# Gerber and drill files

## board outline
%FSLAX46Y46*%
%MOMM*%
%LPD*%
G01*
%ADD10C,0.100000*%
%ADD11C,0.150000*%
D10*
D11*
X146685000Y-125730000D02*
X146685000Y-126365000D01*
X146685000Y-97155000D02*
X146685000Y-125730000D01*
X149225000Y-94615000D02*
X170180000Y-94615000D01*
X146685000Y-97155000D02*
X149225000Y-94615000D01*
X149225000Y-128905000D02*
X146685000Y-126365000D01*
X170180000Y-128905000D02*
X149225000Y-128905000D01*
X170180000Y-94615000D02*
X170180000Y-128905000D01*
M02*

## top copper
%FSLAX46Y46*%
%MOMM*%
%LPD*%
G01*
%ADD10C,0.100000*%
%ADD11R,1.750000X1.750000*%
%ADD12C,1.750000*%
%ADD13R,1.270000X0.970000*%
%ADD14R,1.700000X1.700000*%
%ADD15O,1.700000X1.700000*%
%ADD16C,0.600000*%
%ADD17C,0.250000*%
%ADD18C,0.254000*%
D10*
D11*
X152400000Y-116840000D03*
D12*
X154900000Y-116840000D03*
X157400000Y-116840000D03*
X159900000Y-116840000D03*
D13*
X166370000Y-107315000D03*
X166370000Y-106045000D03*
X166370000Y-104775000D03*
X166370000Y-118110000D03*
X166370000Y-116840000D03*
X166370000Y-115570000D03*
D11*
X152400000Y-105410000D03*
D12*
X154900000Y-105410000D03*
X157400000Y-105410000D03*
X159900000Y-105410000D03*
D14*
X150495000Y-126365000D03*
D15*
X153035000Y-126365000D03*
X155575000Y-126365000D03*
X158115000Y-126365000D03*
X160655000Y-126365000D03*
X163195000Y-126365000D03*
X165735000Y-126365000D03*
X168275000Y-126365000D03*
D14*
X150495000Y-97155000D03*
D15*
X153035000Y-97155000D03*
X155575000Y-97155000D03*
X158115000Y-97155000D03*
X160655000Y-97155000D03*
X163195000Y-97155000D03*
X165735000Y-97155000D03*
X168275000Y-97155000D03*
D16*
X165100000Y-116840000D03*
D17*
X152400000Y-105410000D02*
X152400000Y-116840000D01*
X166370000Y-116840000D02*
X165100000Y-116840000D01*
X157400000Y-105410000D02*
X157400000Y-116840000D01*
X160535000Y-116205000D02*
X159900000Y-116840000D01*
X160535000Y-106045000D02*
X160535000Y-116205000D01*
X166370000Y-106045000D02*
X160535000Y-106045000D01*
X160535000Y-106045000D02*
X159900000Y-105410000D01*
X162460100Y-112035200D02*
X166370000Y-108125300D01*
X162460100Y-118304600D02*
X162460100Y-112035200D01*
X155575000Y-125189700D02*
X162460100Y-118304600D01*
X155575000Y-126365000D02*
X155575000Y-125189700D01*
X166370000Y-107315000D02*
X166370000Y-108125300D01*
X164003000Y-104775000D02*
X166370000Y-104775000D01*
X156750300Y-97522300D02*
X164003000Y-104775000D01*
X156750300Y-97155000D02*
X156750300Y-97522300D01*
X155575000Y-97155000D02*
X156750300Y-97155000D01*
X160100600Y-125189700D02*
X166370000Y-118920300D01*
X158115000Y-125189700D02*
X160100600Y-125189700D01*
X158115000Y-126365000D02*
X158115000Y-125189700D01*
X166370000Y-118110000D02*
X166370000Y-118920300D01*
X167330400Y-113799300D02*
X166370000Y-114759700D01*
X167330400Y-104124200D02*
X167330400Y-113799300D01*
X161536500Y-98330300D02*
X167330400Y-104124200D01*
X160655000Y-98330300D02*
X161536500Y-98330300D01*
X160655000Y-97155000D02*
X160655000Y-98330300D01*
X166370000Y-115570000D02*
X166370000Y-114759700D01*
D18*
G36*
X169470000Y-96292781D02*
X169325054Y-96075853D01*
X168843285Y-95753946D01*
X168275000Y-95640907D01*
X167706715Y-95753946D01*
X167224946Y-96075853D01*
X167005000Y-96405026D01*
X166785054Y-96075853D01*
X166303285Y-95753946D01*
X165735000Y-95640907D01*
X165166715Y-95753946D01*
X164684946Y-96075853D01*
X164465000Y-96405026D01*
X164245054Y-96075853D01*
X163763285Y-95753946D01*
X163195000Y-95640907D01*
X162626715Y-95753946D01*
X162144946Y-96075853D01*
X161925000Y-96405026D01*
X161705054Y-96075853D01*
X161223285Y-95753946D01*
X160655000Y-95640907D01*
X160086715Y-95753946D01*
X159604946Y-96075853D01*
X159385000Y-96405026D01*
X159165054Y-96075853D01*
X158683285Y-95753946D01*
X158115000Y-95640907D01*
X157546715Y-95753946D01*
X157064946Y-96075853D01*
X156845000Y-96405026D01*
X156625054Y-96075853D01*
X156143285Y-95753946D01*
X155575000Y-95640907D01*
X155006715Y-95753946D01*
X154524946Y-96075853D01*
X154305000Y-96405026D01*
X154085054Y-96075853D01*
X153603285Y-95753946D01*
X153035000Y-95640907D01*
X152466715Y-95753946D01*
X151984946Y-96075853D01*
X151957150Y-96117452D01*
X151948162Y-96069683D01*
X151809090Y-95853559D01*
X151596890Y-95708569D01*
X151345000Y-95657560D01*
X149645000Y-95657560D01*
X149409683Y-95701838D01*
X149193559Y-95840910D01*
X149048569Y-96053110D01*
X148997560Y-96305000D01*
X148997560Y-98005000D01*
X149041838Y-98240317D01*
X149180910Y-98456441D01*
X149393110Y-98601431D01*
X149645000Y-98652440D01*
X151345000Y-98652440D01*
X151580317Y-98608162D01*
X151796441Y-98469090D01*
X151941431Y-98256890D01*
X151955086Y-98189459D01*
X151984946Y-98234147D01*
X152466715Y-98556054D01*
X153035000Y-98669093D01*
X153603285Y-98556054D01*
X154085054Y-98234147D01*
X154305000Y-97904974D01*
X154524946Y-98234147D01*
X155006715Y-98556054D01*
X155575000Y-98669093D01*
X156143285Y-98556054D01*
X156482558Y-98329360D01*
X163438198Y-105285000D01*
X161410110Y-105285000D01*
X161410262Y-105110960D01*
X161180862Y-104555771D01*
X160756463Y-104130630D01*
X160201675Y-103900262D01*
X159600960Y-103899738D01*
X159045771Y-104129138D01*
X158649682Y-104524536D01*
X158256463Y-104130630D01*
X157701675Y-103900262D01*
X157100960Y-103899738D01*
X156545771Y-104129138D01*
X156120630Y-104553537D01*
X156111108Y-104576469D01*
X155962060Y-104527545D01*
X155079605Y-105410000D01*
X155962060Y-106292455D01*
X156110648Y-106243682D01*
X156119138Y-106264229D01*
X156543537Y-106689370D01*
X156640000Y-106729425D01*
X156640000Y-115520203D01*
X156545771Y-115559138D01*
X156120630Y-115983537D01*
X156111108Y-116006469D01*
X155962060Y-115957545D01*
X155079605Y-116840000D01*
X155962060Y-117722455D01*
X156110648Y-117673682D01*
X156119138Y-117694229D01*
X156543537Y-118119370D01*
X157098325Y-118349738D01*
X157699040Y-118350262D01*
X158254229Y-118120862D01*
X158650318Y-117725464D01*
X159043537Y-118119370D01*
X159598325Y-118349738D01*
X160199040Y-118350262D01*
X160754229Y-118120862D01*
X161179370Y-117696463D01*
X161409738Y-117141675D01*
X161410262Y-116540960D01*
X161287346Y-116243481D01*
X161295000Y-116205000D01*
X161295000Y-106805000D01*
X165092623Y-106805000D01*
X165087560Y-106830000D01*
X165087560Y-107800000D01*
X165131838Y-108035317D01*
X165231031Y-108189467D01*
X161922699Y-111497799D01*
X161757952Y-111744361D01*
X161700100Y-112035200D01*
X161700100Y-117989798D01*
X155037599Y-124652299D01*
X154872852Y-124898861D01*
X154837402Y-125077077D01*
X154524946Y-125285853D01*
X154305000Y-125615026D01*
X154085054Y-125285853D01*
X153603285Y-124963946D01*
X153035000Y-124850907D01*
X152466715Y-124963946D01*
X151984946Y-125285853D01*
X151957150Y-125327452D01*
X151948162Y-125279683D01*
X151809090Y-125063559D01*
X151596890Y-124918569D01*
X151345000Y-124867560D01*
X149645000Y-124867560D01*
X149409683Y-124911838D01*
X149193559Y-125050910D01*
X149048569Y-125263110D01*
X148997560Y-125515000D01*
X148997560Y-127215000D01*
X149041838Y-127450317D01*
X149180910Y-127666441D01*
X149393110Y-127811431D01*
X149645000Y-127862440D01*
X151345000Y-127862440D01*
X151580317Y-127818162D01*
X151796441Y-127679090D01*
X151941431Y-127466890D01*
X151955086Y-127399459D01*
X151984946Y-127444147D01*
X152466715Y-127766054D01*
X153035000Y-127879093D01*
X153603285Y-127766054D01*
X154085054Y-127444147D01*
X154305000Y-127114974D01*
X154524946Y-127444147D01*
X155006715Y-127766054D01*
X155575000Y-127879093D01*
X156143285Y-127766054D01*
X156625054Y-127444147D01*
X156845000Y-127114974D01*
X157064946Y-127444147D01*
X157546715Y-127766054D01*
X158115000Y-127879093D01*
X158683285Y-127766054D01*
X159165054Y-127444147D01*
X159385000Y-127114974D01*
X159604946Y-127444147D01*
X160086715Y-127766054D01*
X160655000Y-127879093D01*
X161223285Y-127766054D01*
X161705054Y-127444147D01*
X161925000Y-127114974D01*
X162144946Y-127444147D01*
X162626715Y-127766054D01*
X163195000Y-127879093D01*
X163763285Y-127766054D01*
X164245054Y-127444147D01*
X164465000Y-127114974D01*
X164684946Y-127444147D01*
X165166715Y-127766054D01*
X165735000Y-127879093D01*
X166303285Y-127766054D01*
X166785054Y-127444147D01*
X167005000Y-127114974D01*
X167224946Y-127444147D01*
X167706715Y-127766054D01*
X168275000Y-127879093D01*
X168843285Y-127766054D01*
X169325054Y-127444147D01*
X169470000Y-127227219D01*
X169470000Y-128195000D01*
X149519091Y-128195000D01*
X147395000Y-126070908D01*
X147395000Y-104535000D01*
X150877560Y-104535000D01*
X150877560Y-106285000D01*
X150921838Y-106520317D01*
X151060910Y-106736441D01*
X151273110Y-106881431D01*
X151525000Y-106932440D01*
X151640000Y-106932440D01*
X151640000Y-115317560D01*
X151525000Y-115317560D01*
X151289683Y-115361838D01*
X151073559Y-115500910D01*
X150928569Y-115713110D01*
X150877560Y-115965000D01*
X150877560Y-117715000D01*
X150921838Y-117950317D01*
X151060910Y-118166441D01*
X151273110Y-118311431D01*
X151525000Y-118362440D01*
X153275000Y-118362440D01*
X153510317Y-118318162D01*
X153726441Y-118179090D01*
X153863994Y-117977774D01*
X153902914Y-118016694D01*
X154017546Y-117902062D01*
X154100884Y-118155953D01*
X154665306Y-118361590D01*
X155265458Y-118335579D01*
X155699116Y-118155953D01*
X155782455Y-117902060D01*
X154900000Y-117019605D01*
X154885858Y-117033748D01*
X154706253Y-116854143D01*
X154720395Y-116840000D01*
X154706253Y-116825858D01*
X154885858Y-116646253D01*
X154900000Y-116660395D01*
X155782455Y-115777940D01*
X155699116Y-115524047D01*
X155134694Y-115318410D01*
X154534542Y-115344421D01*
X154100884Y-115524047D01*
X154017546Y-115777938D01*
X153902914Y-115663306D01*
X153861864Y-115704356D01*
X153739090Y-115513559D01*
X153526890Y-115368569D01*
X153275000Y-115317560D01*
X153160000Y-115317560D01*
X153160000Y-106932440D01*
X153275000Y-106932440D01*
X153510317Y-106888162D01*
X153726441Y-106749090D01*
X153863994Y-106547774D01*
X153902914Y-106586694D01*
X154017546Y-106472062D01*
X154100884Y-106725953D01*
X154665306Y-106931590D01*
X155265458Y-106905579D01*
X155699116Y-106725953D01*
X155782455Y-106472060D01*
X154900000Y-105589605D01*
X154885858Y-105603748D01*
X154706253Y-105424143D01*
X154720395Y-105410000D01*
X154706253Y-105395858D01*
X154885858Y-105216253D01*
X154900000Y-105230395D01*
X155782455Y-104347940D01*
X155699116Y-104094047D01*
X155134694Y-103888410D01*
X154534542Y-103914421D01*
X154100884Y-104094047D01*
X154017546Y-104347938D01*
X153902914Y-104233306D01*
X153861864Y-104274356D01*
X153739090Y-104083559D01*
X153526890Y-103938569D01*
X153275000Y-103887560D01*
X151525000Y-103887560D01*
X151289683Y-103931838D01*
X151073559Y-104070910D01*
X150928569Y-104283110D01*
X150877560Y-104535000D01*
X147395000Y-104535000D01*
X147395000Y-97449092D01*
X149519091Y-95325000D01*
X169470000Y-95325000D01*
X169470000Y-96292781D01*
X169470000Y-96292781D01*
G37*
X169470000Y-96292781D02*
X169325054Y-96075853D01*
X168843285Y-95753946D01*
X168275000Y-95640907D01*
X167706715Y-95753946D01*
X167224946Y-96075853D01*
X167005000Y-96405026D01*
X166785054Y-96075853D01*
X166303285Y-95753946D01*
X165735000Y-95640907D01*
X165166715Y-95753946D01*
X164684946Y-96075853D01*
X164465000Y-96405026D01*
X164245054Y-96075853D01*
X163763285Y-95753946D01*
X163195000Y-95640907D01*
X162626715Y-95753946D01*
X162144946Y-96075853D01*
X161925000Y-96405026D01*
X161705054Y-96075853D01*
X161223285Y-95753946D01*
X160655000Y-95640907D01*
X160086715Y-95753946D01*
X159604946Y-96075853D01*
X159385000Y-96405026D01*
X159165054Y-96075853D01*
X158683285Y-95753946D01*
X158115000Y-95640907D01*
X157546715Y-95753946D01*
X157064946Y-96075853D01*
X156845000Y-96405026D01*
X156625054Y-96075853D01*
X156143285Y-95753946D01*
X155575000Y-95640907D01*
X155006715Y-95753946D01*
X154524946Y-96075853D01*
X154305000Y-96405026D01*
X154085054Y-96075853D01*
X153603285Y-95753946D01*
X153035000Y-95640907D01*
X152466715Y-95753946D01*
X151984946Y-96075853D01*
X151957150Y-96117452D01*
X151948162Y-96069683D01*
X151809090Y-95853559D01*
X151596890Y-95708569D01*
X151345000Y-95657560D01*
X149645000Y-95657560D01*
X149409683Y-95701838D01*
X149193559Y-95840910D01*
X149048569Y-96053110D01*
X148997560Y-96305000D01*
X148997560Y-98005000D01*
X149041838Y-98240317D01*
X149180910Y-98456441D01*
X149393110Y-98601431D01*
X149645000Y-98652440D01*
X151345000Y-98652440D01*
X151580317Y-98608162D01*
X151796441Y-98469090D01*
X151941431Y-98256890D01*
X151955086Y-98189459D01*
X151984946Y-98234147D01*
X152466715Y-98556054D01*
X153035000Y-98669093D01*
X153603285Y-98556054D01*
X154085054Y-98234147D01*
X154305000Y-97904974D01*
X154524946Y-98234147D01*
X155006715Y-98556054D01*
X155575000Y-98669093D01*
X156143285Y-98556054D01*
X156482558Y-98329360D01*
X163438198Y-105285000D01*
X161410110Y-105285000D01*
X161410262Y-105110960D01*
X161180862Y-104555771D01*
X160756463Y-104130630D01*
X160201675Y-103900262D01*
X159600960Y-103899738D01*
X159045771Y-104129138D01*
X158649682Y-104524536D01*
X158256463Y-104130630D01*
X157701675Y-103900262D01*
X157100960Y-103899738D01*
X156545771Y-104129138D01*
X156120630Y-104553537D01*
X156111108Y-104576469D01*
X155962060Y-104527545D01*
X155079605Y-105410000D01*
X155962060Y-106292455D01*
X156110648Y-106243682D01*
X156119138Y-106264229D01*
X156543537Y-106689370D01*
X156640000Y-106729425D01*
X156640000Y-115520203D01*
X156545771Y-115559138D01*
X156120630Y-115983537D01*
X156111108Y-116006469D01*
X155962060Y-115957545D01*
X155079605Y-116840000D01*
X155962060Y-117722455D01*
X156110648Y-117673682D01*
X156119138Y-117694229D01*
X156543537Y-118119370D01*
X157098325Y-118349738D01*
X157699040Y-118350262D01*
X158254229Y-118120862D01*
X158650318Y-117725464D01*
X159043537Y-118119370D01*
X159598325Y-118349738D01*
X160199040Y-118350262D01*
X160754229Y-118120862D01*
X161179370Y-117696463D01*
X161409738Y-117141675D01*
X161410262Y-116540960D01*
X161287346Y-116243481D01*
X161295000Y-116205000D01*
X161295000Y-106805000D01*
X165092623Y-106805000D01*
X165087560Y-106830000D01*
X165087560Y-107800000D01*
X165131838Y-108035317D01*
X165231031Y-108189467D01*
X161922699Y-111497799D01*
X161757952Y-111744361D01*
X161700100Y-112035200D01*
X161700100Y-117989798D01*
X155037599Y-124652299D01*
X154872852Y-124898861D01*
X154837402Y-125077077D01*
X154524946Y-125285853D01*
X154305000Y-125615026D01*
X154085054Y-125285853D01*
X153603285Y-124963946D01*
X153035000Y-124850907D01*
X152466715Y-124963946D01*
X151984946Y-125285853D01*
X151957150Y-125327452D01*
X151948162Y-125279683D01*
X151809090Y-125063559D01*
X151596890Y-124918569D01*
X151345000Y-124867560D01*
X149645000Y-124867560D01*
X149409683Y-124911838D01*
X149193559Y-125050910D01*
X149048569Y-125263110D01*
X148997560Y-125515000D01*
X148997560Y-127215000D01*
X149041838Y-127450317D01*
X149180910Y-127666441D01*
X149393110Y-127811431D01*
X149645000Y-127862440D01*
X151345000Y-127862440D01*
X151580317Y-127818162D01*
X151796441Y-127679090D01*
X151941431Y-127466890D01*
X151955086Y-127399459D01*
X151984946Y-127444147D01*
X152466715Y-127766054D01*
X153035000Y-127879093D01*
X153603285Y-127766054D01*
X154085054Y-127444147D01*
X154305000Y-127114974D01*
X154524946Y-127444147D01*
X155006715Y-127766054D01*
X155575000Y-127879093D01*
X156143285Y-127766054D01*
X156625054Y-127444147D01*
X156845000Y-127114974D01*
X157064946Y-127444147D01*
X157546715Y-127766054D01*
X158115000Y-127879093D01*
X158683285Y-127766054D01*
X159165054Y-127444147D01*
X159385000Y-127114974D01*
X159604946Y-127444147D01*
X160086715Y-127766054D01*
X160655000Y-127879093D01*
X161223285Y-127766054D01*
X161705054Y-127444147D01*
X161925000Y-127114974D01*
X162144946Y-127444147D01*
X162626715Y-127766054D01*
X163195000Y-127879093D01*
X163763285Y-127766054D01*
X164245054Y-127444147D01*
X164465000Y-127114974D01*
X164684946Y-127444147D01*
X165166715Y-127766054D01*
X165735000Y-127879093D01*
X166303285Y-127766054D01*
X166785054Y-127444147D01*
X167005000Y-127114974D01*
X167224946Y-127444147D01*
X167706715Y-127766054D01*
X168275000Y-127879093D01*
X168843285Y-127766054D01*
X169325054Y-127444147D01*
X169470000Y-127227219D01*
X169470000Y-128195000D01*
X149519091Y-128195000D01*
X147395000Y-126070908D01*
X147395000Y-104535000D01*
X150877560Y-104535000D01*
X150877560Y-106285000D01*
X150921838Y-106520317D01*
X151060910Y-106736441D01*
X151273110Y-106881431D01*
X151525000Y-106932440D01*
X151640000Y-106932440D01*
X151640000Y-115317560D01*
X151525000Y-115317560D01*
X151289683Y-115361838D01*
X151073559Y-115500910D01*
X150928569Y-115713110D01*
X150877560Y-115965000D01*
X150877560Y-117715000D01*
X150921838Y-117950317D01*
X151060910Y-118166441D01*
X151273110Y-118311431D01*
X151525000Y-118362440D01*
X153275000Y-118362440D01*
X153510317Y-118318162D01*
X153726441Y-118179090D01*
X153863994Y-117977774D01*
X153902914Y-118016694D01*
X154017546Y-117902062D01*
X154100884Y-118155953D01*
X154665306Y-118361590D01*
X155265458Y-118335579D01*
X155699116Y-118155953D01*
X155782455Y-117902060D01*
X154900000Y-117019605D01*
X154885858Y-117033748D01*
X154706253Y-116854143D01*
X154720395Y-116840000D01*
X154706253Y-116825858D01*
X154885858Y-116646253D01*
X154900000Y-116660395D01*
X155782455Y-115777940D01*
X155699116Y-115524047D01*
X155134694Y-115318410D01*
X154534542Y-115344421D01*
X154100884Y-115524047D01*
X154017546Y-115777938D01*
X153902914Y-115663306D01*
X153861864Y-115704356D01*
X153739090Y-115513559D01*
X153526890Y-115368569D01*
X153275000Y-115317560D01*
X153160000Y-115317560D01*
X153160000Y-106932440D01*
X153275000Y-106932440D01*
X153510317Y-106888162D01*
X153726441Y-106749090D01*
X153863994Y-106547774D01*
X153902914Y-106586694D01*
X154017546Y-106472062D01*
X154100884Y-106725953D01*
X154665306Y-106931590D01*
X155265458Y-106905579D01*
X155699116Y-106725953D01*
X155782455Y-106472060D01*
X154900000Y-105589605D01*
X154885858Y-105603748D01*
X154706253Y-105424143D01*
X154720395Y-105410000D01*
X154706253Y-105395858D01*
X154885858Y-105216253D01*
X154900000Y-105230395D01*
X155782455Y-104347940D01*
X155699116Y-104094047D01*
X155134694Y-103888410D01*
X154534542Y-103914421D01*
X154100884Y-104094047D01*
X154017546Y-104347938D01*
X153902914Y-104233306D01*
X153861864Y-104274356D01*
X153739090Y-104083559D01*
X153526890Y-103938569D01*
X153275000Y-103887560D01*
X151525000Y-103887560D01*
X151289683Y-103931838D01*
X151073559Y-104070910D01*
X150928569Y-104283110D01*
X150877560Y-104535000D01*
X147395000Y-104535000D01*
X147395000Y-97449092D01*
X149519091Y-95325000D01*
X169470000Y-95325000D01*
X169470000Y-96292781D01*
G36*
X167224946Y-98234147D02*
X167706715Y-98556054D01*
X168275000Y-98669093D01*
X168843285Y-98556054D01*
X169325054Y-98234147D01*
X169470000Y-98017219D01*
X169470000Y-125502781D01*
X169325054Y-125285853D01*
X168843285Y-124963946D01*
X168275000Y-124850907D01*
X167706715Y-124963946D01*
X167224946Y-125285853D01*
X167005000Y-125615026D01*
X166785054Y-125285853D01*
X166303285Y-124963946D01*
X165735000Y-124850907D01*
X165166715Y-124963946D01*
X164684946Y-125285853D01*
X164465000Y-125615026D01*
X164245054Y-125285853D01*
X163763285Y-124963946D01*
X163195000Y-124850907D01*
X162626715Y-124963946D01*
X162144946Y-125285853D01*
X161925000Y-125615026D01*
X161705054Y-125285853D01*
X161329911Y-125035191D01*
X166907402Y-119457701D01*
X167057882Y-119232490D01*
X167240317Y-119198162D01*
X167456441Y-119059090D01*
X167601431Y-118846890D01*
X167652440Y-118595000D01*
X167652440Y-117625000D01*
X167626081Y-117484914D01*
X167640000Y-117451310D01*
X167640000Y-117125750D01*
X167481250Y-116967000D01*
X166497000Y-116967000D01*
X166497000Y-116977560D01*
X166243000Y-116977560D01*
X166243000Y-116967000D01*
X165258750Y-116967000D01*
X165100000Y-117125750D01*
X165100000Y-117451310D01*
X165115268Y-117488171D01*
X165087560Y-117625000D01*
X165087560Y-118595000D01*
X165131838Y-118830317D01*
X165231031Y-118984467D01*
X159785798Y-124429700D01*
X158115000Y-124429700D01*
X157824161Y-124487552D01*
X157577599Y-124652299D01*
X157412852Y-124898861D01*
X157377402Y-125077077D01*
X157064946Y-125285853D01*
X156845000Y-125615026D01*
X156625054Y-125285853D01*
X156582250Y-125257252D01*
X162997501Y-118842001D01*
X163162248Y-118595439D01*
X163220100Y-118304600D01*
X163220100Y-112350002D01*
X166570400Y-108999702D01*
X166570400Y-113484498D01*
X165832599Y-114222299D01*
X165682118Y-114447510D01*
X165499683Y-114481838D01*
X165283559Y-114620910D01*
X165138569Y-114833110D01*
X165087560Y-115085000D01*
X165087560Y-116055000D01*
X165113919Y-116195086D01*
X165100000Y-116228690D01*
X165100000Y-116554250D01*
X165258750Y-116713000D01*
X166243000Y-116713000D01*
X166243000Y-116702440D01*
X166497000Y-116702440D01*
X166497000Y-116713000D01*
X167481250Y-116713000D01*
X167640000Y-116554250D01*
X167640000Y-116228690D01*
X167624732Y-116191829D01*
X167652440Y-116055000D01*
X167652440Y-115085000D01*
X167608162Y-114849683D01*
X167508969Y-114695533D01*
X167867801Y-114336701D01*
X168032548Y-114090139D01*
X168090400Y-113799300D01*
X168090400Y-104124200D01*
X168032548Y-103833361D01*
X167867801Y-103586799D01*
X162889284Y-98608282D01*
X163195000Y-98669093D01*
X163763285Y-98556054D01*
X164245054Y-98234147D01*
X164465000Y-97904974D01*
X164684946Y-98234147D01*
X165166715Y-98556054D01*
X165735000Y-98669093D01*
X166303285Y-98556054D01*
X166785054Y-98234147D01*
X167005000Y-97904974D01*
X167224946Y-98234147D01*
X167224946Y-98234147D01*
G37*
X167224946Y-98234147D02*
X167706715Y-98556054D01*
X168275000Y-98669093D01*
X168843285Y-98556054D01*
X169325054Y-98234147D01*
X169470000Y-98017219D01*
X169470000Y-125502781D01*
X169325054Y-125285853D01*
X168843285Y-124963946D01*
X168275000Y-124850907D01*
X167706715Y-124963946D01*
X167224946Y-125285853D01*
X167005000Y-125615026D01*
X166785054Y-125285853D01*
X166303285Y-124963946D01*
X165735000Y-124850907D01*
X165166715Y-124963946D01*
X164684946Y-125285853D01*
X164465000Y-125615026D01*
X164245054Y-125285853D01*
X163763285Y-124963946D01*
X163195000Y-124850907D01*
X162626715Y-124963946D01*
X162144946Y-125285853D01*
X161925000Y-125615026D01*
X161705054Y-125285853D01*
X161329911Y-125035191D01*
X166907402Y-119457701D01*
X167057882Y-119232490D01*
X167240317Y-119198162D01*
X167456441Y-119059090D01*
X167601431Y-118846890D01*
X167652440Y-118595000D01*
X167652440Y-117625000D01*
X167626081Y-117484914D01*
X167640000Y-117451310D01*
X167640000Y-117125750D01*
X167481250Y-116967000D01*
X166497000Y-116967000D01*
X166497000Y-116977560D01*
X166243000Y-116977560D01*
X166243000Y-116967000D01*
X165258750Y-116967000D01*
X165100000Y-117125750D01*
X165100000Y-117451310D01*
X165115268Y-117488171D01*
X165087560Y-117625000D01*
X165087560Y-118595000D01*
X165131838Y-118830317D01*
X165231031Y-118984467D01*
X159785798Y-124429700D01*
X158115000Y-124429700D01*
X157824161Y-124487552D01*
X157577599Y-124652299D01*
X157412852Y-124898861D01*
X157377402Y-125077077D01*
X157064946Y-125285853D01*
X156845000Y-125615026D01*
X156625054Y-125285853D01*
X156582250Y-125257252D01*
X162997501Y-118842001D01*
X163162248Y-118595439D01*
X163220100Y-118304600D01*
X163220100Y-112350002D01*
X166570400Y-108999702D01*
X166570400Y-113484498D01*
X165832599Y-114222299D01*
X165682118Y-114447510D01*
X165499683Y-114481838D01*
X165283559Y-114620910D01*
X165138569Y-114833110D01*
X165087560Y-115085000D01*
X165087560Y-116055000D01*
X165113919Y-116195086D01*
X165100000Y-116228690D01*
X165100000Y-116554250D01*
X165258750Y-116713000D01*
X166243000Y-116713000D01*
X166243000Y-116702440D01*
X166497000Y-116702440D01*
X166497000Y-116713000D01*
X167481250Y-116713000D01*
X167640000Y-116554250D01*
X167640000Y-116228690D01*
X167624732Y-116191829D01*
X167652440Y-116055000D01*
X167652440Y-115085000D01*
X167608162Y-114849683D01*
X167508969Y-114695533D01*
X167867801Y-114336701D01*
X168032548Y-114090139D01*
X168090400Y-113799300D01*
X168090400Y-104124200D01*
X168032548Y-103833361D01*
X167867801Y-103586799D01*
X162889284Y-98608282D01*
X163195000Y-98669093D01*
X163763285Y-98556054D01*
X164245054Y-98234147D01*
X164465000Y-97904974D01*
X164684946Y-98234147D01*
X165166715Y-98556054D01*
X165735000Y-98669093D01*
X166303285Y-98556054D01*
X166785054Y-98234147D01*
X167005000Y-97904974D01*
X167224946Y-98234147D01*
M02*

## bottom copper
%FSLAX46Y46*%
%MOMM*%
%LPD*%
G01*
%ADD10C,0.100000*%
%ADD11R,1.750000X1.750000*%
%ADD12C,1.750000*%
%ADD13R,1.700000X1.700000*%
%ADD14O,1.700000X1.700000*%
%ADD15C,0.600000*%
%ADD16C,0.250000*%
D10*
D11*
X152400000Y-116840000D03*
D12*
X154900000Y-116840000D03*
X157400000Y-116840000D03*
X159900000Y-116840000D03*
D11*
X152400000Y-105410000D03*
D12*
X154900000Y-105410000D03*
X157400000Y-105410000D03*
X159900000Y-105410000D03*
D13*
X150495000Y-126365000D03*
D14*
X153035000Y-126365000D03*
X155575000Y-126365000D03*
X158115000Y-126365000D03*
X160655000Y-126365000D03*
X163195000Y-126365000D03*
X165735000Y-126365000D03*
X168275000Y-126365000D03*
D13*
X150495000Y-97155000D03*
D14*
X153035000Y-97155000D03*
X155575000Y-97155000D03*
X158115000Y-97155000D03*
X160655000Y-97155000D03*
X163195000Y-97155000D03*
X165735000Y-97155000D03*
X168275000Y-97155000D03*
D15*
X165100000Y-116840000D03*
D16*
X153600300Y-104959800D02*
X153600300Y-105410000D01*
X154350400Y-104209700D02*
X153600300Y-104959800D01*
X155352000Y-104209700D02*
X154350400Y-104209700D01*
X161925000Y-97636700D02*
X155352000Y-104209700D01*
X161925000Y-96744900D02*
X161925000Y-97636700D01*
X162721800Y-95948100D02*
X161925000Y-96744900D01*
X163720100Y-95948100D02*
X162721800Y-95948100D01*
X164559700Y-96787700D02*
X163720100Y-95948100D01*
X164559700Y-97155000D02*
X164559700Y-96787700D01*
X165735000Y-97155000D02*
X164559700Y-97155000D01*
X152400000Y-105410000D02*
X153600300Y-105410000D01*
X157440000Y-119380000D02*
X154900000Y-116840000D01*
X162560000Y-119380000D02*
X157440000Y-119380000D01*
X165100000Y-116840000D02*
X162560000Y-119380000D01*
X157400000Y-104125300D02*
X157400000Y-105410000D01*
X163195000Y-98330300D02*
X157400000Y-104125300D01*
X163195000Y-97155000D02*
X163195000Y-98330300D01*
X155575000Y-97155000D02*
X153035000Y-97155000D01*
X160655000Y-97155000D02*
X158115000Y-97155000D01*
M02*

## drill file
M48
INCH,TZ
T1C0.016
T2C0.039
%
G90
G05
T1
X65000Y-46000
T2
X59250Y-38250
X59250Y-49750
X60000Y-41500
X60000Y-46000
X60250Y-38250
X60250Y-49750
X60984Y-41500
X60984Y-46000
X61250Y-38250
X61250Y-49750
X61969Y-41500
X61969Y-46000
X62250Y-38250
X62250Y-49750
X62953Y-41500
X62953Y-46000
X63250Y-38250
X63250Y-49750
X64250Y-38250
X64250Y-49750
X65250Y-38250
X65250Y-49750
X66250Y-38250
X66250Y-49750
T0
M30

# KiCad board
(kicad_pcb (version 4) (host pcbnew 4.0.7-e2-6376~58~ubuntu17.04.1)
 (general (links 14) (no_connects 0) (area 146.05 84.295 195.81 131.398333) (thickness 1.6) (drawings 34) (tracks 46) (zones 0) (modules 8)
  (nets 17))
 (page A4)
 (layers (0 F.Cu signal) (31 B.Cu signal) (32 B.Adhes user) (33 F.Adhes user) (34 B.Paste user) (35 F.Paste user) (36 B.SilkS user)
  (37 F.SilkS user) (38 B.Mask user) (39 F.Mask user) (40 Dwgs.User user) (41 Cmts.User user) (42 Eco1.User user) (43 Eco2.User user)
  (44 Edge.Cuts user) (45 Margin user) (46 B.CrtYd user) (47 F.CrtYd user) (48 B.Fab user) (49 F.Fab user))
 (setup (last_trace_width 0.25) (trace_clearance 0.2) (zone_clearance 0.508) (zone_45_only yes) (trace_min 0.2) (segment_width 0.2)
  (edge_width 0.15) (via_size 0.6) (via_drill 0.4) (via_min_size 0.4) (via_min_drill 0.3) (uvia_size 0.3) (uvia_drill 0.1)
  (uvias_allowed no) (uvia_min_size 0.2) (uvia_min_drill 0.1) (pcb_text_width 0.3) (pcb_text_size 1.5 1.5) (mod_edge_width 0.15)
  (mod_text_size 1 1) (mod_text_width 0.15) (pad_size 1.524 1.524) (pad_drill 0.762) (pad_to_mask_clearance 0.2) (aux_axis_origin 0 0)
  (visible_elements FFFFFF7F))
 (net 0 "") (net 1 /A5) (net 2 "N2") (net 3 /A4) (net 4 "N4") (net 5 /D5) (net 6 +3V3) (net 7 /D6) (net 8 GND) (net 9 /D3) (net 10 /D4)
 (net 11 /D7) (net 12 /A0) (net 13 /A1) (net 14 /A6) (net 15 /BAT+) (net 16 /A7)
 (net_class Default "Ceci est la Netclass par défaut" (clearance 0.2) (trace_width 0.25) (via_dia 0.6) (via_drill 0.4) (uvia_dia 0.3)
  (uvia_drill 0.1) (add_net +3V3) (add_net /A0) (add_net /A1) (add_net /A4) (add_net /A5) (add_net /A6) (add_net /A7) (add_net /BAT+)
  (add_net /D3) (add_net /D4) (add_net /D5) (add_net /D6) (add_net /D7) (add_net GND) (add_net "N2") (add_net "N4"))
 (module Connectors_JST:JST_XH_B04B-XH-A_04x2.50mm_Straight (layer F.Cu) (at 152.4 116.84)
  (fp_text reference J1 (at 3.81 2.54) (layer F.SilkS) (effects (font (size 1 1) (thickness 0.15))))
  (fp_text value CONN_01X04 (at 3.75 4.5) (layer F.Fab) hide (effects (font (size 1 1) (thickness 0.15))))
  (pad 1 thru_hole rect (at 0 0) (size 1.75 1.75) (drill 1) (layers *.Cu *.Mask) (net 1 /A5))
  (pad 2 thru_hole circle (at 2.5 0) (size 1.75 1.75) (drill 1) (layers *.Cu *.Mask) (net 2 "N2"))
  (pad 3 thru_hole circle (at 5 0) (size 1.75 1.75) (drill 1) (layers *.Cu *.Mask) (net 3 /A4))
  (pad 4 thru_hole circle (at 7.5 0) (size 1.75 1.75) (drill 1) (layers *.Cu *.Mask) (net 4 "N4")))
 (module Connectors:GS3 (layer F.Cu) (at 166.37 106.045 180)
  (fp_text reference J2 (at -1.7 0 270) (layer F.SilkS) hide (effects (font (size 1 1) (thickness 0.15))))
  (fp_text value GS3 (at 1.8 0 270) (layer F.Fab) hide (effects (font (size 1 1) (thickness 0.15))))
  (pad 1 smd rect (at 0 -1.27 180) (size 1.27 0.97) (layers F.Cu F.Paste F.Mask) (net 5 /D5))
  (pad 2 smd rect (at 0 0 180) (size 1.27 0.97) (layers F.Cu F.Paste F.Mask) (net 4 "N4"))
  (pad 3 smd rect (at 0 1.27 180) (size 1.27 0.97) (layers F.Cu F.Paste F.Mask) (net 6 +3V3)))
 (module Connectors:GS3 (layer F.Cu) (at 166.37 116.84 180)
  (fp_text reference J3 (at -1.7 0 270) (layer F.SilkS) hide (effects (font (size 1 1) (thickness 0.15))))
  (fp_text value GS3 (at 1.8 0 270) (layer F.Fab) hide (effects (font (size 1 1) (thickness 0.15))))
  (pad 1 smd rect (at 0 -1.27 180) (size 1.27 0.97) (layers F.Cu F.Paste F.Mask) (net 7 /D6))
  (pad 2 smd rect (at 0 0 180) (size 1.27 0.97) (layers F.Cu F.Paste F.Mask) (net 2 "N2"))
  (pad 3 smd rect (at 0 1.27 180) (size 1.27 0.97) (layers F.Cu F.Paste F.Mask) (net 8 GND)))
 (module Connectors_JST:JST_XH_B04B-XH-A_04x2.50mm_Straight (layer F.Cu) (at 152.4 105.41)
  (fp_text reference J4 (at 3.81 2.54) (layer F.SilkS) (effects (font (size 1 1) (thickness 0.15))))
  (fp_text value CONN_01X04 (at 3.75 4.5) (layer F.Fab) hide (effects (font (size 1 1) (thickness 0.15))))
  (pad 1 thru_hole rect (at 0 0) (size 1.75 1.75) (drill 1) (layers *.Cu *.Mask) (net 1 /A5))
  (pad 2 thru_hole circle (at 2.5 0) (size 1.75 1.75) (drill 1) (layers *.Cu *.Mask) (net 2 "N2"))
  (pad 3 thru_hole circle (at 5 0) (size 1.75 1.75) (drill 1) (layers *.Cu *.Mask) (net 3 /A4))
  (pad 4 thru_hole circle (at 7.5 0) (size 1.75 1.75) (drill 1) (layers *.Cu *.Mask) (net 4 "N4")))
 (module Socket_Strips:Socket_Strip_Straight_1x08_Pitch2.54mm (layer B.Cu) (at 150.495 126.365 270)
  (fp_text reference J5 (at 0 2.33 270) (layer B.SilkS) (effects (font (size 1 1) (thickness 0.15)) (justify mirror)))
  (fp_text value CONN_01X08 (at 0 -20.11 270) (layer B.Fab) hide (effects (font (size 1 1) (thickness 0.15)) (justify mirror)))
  (pad 1 thru_hole rect (at 0 0 270) (size 1.7 1.7) (drill 1) (layers *.Cu *.Mask) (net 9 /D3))
  (pad 2 thru_hole oval (at 0 -2.54 270) (size 1.7 1.7) (drill 1) (layers *.Cu *.Mask) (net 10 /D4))
  (pad 3 thru_hole oval (at 0 -5.08 270) (size 1.7 1.7) (drill 1) (layers *.Cu *.Mask) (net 5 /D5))
  (pad 4 thru_hole oval (at 0 -7.62 270) (size 1.7 1.7) (drill 1) (layers *.Cu *.Mask) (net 7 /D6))
  (pad 5 thru_hole oval (at 0 -10.16 270) (size 1.7 1.7) (drill 1) (layers *.Cu *.Mask) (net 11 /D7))
  (pad 6 thru_hole oval (at 0 -12.7 270) (size 1.7 1.7) (drill 1) (layers *.Cu *.Mask) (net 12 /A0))
  (pad 7 thru_hole oval (at 0 -15.24 270) (size 1.7 1.7) (drill 1) (layers *.Cu *.Mask) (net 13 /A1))
  (pad 8 thru_hole oval (at 0 -17.78 270) (size 1.7 1.7) (drill 1) (layers *.Cu *.Mask) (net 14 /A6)))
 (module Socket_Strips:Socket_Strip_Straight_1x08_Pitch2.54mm (layer B.Cu) (at 150.495 97.155 270)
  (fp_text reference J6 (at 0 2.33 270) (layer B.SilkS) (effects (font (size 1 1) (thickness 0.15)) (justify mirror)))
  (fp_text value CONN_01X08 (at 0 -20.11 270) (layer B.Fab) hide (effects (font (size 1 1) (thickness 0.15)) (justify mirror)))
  (pad 1 thru_hole rect (at 0 0 270) (size 1.7 1.7) (drill 1) (layers *.Cu *.Mask) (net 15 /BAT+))
  (pad 2 thru_hole oval (at 0 -2.54 270) (size 1.7 1.7) (drill 1) (layers *.Cu *.Mask) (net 6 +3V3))
  (pad 3 thru_hole oval (at 0 -5.08 270) (size 1.7 1.7) (drill 1) (layers *.Cu *.Mask) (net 6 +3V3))
  (pad 4 thru_hole oval (at 0 -7.62 270) (size 1.7 1.7) (drill 1) (layers *.Cu *.Mask) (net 8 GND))
  (pad 5 thru_hole oval (at 0 -10.16 270) (size 1.7 1.7) (drill 1) (layers *.Cu *.Mask) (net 8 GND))
  (pad 6 thru_hole oval (at 0 -12.7 270) (size 1.7 1.7) (drill 1) (layers *.Cu *.Mask) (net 3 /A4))
  (pad 7 thru_hole oval (at 0 -15.24 270) (size 1.7 1.7) (drill 1) (layers *.Cu *.Mask) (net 1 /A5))
  (pad 8 thru_hole oval (at 0 -17.78 270) (size 1.7 1.7) (drill 1) (layers *.Cu *.Mask) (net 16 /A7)))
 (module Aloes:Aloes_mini (layer F.Cu) (at 149.225 122.555 90)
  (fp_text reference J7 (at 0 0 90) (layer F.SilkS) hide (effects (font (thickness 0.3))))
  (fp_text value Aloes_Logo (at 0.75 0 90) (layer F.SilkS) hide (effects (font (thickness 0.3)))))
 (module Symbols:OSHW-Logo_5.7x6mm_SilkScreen (layer B.Cu) (at 151.765 101.6 270)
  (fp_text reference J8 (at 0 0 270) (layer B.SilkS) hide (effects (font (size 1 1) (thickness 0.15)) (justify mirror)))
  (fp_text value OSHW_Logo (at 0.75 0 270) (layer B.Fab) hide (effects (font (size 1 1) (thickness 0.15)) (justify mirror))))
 (gr_line (start 146.685 125.73) (end 146.685 126.365) (angle 90) (layer Edge.Cuts) (width 0.15))
 (gr_line (start 146.685 97.155) (end 146.685 125.73) (angle 90) (layer Edge.Cuts) (width 0.15))
 (gr_line (start 149.225 94.615) (end 170.18 94.615) (angle 90) (layer Edge.Cuts) (width 0.15))
 (gr_line (start 146.685 97.155) (end 149.225 94.615) (angle 90) (layer Edge.Cuts) (width 0.15))
 (gr_line (start 149.225 128.905) (end 146.685 126.365) (angle 90) (layer Edge.Cuts) (width 0.15))
 (gr_line (start 170.18 128.905) (end 149.225 128.905) (angle 90) (layer Edge.Cuts) (width 0.15))
 (gr_line (start 170.18 94.615) (end 170.18 128.905) (angle 90) (layer Edge.Cuts) (width 0.15))
 (segment (start 152.4 105.41) (end 152.4 116.84) (width 0.25) (layer F.Cu) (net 1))
 (segment (start 153.6003 104.9598) (end 153.6003 105.41) (width 0.25) (layer B.Cu) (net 1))
 (segment (start 154.3504 104.2097) (end 153.6003 104.9598) (width 0.25) (layer B.Cu) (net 1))
 (segment (start 155.352 104.2097) (end 154.3504 104.2097) (width 0.25) (layer B.Cu) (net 1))
 (segment (start 161.925 97.6367) (end 155.352 104.2097) (width 0.25) (layer B.Cu) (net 1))
 (segment (start 161.925 96.7449) (end 161.925 97.6367) (width 0.25) (layer B.Cu) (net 1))
 (segment (start 162.7218 95.9481) (end 161.925 96.7449) (width 0.25) (layer B.Cu) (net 1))
 (segment (start 163.7201 95.9481) (end 162.7218 95.9481) (width 0.25) (layer B.Cu) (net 1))
 (segment (start 164.5597 96.7877) (end 163.7201 95.9481) (width 0.25) (layer B.Cu) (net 1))
 (segment (start 164.5597 97.155) (end 164.5597 96.7877) (width 0.25) (layer B.Cu) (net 1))
 (segment (start 165.735 97.155) (end 164.5597 97.155) (width 0.25) (layer B.Cu) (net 1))
 (segment (start 152.4 105.41) (end 153.6003 105.41) (width 0.25) (layer B.Cu) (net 1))
 (segment (start 166.37 116.84) (end 165.1 116.84) (width 0.25) (layer F.Cu) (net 2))
 (segment (start 157.44 119.38) (end 154.9 116.84) (width 0.25) (layer B.Cu) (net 2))
 (segment (start 162.56 119.38) (end 157.44 119.38) (width 0.25) (layer B.Cu) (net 2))
 (segment (start 165.1 116.84) (end 162.56 119.38) (width 0.25) (layer B.Cu) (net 2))
 (via (at 165.1 116.84) (size 0.6) (drill 0.4) (layers F.Cu B.Cu) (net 2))
 (segment (start 157.4 105.41) (end 157.4 116.84) (width 0.25) (layer F.Cu) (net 3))
 (segment (start 157.4 104.1253) (end 157.4 105.41) (width 0.25) (layer B.Cu) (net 3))
 (segment (start 163.195 98.3303) (end 157.4 104.1253) (width 0.25) (layer B.Cu) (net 3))
 (segment (start 163.195 97.155) (end 163.195 98.3303) (width 0.25) (layer B.Cu) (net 3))
 (segment (start 160.535 116.205) (end 159.9 116.84) (width 0.25) (layer F.Cu) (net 4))
 (segment (start 160.535 106.045) (end 160.535 116.205) (width 0.25) (layer F.Cu) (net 4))
 (segment (start 166.37 106.045) (end 160.535 106.045) (width 0.25) (layer F.Cu) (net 4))
 (segment (start 160.535 106.045) (end 159.9 105.41) (width 0.25) (layer F.Cu) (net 4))
 (segment (start 162.4601 112.0352) (end 166.37 108.1253) (width 0.25) (layer F.Cu) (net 5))
 (segment (start 162.4601 118.3046) (end 162.4601 112.0352) (width 0.25) (layer F.Cu) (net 5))
 (segment (start 155.575 125.1897) (end 162.4601 118.3046) (width 0.25) (layer F.Cu) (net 5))
 (segment (start 155.575 126.365) (end 155.575 125.1897) (width 0.25) (layer F.Cu) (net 5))
 (segment (start 166.37 107.315) (end 166.37 108.1253) (width 0.25) (layer F.Cu) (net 5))
 (segment (start 155.575 97.155) (end 153.035 97.155) (width 0.25) (layer B.Cu) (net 6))
 (segment (start 164.003 104.775) (end 166.37 104.775) (width 0.25) (layer F.Cu) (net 6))
 (segment (start 156.7503 97.5223) (end 164.003 104.775) (width 0.25) (layer F.Cu) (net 6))
 (segment (start 156.7503 97.155) (end 156.7503 97.5223) (width 0.25) (layer F.Cu) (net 6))
 (segment (start 155.575 97.155) (end 156.7503 97.155) (width 0.25) (layer F.Cu) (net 6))
 (segment (start 160.1006 125.1897) (end 166.37 118.9203) (width 0.25) (layer F.Cu) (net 7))
 (segment (start 158.115 125.1897) (end 160.1006 125.1897) (width 0.25) (layer F.Cu) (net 7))
 (segment (start 158.115 126.365) (end 158.115 125.1897) (width 0.25) (layer F.Cu) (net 7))
 (segment (start 166.37 118.11) (end 166.37 118.9203) (width 0.25) (layer F.Cu) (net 7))
 (segment (start 160.655 97.155) (end 158.115 97.155) (width 0.25) (layer B.Cu) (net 8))
 (segment (start 167.3304 113.7993) (end 166.37 114.7597) (width 0.25) (layer F.Cu) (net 8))
 (segment (start 167.3304 104.1242) (end 167.3304 113.7993) (width 0.25) (layer F.Cu) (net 8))
 (segment (start 161.5365 98.3303) (end 167.3304 104.1242) (width 0.25) (layer F.Cu) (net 8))
 (segment (start 160.655 98.3303) (end 161.5365 98.3303) (width 0.25) (layer F.Cu) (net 8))
 (segment (start 160.655 97.155) (end 160.655 98.3303) (width 0.25) (layer F.Cu) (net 8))
 (segment (start 166.37 115.57) (end 166.37 114.7597) (width 0.25) (layer F.Cu) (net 8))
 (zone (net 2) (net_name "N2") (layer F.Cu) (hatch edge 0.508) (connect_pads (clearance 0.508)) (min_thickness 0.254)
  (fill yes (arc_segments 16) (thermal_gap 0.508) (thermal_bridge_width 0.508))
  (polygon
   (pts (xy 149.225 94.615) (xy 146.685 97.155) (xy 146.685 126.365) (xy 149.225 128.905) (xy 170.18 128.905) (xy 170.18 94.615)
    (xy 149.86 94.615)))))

